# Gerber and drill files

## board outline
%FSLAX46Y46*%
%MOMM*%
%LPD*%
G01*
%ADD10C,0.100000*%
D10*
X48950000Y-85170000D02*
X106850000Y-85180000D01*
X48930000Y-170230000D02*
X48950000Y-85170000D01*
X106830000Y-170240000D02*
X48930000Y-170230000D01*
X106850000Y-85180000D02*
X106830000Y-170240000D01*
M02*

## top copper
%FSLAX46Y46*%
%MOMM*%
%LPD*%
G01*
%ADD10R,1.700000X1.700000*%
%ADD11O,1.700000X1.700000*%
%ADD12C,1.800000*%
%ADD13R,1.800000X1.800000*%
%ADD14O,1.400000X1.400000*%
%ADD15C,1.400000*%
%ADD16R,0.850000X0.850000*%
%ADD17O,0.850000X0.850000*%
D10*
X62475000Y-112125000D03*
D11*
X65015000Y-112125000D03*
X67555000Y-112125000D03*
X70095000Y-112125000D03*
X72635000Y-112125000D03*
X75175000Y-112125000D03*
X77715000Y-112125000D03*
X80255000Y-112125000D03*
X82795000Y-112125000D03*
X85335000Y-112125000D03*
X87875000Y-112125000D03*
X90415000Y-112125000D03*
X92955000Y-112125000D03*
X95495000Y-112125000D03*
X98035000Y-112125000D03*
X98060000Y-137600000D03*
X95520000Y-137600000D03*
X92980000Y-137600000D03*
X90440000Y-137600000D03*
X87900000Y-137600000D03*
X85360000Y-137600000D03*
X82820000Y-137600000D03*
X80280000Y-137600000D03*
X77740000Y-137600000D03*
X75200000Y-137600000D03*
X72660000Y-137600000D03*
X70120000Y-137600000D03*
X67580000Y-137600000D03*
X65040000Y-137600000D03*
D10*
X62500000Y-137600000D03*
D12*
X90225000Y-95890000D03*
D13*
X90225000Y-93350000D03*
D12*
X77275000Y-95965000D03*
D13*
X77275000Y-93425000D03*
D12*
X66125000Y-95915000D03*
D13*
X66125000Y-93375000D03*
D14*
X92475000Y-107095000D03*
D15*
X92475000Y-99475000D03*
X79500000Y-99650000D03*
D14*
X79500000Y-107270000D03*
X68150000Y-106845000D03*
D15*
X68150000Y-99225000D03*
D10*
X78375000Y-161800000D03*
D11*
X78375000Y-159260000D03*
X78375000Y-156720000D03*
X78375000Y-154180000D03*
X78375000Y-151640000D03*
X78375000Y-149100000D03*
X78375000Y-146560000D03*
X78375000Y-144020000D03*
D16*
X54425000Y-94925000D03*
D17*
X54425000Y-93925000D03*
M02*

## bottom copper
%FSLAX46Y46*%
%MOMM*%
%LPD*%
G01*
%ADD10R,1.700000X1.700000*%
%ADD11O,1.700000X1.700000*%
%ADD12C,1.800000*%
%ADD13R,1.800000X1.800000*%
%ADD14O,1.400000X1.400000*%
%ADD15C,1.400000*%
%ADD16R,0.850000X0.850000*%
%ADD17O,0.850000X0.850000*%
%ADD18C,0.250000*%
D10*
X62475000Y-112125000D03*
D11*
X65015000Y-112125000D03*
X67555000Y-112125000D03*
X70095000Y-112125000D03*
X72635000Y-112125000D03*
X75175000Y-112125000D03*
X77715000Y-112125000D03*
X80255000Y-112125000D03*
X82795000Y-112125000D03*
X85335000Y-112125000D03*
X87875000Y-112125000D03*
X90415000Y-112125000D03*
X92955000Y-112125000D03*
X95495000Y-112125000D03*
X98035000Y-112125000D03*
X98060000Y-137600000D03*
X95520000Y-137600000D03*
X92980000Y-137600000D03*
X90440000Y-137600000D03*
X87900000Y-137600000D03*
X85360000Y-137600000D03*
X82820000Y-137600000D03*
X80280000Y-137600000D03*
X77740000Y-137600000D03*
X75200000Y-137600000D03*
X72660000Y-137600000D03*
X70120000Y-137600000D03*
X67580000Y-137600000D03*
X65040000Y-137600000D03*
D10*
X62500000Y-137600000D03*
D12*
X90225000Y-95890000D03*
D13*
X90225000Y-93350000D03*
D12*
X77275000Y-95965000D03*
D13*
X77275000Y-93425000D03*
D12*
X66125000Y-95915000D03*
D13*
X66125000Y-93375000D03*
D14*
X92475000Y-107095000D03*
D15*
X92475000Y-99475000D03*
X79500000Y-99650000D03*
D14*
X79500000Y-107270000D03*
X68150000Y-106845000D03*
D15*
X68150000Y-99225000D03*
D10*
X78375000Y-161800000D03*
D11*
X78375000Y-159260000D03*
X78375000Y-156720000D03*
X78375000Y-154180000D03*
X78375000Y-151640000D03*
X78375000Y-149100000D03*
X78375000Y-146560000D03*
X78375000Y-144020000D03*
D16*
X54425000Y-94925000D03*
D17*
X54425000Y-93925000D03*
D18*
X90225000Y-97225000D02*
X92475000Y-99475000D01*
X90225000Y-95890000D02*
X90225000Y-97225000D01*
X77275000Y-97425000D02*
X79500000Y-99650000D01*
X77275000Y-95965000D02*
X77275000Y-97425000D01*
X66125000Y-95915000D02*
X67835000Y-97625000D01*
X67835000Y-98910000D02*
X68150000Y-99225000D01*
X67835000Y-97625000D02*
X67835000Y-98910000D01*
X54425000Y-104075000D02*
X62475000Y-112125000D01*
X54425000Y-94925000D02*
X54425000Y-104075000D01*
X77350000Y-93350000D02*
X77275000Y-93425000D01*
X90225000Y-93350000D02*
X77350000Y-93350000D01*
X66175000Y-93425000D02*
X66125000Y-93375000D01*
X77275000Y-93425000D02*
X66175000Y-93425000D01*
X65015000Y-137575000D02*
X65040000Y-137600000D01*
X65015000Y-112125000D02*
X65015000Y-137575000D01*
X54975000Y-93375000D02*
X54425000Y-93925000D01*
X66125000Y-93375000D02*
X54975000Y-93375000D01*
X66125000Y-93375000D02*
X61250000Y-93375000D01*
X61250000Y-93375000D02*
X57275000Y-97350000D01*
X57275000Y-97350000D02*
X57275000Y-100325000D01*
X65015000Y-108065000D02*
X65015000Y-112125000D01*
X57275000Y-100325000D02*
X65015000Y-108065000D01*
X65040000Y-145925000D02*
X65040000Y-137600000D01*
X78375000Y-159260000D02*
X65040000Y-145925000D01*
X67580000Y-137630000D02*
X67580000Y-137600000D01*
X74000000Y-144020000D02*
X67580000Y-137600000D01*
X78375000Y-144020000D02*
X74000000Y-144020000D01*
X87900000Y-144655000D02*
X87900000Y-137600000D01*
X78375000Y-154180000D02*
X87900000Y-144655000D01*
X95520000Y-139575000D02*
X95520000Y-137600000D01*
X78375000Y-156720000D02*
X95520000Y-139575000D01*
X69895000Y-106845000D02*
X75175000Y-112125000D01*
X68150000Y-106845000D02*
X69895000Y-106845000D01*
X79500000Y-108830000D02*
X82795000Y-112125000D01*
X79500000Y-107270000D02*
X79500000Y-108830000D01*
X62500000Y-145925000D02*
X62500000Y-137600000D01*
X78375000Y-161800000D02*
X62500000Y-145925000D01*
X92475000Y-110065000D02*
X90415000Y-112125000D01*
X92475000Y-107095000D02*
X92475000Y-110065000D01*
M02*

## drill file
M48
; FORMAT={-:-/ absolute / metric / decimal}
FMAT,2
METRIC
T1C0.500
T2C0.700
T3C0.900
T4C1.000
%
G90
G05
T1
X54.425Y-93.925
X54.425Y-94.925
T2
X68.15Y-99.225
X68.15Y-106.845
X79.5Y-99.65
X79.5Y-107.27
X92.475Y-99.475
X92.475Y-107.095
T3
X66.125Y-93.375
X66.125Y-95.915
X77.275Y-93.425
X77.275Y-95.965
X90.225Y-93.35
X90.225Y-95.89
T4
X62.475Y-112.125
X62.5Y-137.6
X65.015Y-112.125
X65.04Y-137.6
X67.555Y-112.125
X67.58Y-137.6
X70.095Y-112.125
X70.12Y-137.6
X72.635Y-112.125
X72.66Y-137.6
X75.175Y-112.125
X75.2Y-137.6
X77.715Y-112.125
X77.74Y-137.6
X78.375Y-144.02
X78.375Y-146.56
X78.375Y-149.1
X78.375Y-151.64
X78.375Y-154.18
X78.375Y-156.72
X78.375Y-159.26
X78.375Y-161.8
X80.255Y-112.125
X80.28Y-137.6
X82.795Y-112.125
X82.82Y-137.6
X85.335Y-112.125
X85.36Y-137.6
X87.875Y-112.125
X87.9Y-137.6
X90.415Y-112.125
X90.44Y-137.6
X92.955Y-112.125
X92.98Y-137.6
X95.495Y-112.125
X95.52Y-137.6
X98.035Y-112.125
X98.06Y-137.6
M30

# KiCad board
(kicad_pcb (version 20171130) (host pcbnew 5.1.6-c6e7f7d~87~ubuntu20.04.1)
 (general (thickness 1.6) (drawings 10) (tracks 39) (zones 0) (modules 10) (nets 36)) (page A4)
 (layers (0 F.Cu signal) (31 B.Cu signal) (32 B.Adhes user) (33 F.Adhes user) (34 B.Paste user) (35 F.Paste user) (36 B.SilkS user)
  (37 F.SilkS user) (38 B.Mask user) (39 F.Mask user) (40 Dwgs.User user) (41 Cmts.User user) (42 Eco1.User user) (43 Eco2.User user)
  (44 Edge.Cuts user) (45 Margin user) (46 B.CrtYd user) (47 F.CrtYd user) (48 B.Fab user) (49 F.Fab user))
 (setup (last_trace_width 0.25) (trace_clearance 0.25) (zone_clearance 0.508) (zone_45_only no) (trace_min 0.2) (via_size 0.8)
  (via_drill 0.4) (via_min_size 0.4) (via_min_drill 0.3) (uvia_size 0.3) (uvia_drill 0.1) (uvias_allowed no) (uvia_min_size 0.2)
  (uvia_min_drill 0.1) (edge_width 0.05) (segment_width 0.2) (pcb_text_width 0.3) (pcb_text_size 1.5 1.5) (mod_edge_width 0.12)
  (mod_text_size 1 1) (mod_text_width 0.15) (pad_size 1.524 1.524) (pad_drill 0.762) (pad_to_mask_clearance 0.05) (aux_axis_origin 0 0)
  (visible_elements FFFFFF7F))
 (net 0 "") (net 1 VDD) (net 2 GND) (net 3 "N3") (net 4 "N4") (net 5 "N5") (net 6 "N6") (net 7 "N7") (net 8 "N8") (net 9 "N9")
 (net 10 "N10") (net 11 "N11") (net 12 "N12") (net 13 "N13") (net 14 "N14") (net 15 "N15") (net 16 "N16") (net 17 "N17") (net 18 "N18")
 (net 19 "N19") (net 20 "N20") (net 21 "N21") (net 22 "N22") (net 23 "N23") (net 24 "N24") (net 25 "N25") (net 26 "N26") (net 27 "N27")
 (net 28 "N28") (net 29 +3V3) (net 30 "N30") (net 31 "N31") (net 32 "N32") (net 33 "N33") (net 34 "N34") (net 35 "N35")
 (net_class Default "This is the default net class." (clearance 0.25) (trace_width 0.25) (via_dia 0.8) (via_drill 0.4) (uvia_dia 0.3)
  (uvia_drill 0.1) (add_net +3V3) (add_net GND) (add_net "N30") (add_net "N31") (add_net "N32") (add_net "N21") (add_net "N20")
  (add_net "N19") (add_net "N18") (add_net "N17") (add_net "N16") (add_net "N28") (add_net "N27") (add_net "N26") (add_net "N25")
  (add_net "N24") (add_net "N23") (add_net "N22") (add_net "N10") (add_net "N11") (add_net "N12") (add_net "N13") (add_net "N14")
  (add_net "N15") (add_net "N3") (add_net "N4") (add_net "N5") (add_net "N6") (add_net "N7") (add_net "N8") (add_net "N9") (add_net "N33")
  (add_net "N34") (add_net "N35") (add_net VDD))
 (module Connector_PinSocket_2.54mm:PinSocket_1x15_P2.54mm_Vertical (layer F.Cu) (at 62.475 112.125 90)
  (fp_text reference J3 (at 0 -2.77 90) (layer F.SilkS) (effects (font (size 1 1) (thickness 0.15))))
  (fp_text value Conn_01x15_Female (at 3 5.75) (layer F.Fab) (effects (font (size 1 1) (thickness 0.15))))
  (pad 1 thru_hole rect (at 0 0 90) (size 1.7 1.7) (drill 1) (layers *.Cu *.Mask) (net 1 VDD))
  (pad 2 thru_hole oval (at 0 2.54 90) (size 1.7 1.7) (drill 1) (layers *.Cu *.Mask) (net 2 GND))
  (pad 3 thru_hole oval (at 0 5.08 90) (size 1.7 1.7) (drill 1) (layers *.Cu *.Mask) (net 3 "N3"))
  (pad 4 thru_hole oval (at 0 7.62 90) (size 1.7 1.7) (drill 1) (layers *.Cu *.Mask) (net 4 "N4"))
  (pad 5 thru_hole oval (at 0 10.16 90) (size 1.7 1.7) (drill 1) (layers *.Cu *.Mask) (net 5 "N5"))
  (pad 6 thru_hole oval (at 0 12.7 90) (size 1.7 1.7) (drill 1) (layers *.Cu *.Mask) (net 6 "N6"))
  (pad 7 thru_hole oval (at 0 15.24 90) (size 1.7 1.7) (drill 1) (layers *.Cu *.Mask) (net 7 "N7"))
  (pad 8 thru_hole oval (at 0 17.78 90) (size 1.7 1.7) (drill 1) (layers *.Cu *.Mask) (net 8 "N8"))
  (pad 9 thru_hole oval (at 0 20.32 90) (size 1.7 1.7) (drill 1) (layers *.Cu *.Mask) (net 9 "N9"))
  (pad 10 thru_hole oval (at 0 22.86 90) (size 1.7 1.7) (drill 1) (layers *.Cu *.Mask) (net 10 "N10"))
  (pad 11 thru_hole oval (at 0 25.4 90) (size 1.7 1.7) (drill 1) (layers *.Cu *.Mask) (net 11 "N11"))
  (pad 12 thru_hole oval (at 0 27.94 90) (size 1.7 1.7) (drill 1) (layers *.Cu *.Mask) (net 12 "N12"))
  (pad 13 thru_hole oval (at 0 30.48 90) (size 1.7 1.7) (drill 1) (layers *.Cu *.Mask) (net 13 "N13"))
  (pad 14 thru_hole oval (at 0 33.02 90) (size 1.7 1.7) (drill 1) (layers *.Cu *.Mask) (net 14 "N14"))
  (pad 15 thru_hole oval (at 0 35.56 90) (size 1.7 1.7) (drill 1) (layers *.Cu *.Mask) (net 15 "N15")))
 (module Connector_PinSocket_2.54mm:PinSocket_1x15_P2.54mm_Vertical (layer F.Cu) (at 62.5 137.6 90)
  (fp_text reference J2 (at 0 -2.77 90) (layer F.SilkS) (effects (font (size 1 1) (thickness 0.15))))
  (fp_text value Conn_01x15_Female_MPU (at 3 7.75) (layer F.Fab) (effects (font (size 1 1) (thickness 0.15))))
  (pad 15 thru_hole oval (at 0 35.56 90) (size 1.7 1.7) (drill 1) (layers *.Cu *.Mask) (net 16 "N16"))
  (pad 14 thru_hole oval (at 0 33.02 90) (size 1.7 1.7) (drill 1) (layers *.Cu *.Mask) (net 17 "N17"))
  (pad 13 thru_hole oval (at 0 30.48 90) (size 1.7 1.7) (drill 1) (layers *.Cu *.Mask) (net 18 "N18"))
  (pad 12 thru_hole oval (at 0 27.94 90) (size 1.7 1.7) (drill 1) (layers *.Cu *.Mask) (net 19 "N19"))
  (pad 11 thru_hole oval (at 0 25.4 90) (size 1.7 1.7) (drill 1) (layers *.Cu *.Mask) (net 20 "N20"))
  (pad 10 thru_hole oval (at 0 22.86 90) (size 1.7 1.7) (drill 1) (layers *.Cu *.Mask) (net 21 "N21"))
  (pad 9 thru_hole oval (at 0 20.32 90) (size 1.7 1.7) (drill 1) (layers *.Cu *.Mask) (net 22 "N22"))
  (pad 8 thru_hole oval (at 0 17.78 90) (size 1.7 1.7) (drill 1) (layers *.Cu *.Mask) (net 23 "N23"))
  (pad 7 thru_hole oval (at 0 15.24 90) (size 1.7 1.7) (drill 1) (layers *.Cu *.Mask) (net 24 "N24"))
  (pad 6 thru_hole oval (at 0 12.7 90) (size 1.7 1.7) (drill 1) (layers *.Cu *.Mask) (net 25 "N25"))
  (pad 5 thru_hole oval (at 0 10.16 90) (size 1.7 1.7) (drill 1) (layers *.Cu *.Mask) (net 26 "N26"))
  (pad 4 thru_hole oval (at 0 7.62 90) (size 1.7 1.7) (drill 1) (layers *.Cu *.Mask) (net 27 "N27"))
  (pad 3 thru_hole oval (at 0 5.08 90) (size 1.7 1.7) (drill 1) (layers *.Cu *.Mask) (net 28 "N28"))
  (pad 2 thru_hole oval (at 0 2.54 90) (size 1.7 1.7) (drill 1) (layers *.Cu *.Mask) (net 2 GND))
  (pad 1 thru_hole rect (at 0 0 90) (size 1.7 1.7) (drill 1) (layers *.Cu *.Mask) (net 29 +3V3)))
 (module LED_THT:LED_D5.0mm (layer F.Cu) (at 90.225 93.35 270)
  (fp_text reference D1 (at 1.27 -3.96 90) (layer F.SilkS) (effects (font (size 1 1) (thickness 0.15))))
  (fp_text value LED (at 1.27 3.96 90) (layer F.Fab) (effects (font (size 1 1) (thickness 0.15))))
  (pad 2 thru_hole circle (at 2.54 0 270) (size 1.8 1.8) (drill 0.9) (layers *.Cu *.Mask) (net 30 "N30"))
  (pad 1 thru_hole rect (at 0 0 270) (size 1.8 1.8) (drill 0.9) (layers *.Cu *.Mask) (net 2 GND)))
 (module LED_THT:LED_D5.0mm (layer F.Cu) (at 77.275 93.425 270)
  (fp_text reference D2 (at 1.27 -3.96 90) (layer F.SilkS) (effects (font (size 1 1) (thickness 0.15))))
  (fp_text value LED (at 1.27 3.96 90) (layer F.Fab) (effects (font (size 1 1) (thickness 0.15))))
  (pad 2 thru_hole circle (at 2.54 0 270) (size 1.8 1.8) (drill 0.9) (layers *.Cu *.Mask) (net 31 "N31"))
  (pad 1 thru_hole rect (at 0 0 270) (size 1.8 1.8) (drill 0.9) (layers *.Cu *.Mask) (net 2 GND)))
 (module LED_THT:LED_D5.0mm (layer F.Cu) (at 66.125 93.375 270)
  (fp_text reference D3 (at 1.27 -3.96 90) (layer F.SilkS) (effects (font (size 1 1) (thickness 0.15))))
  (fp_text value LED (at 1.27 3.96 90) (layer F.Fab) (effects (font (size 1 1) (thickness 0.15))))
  (pad 2 thru_hole circle (at 2.54 0 270) (size 1.8 1.8) (drill 0.9) (layers *.Cu *.Mask) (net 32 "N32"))
  (pad 1 thru_hole rect (at 0 0 270) (size 1.8 1.8) (drill 0.9) (layers *.Cu *.Mask) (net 2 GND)))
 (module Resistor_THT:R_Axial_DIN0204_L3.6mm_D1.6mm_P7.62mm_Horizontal (layer F.Cu) (at 92.475 99.475 270)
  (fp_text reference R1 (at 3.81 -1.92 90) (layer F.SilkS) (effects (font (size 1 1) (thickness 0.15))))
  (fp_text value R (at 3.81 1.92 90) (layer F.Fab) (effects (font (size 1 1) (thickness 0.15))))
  (pad 2 thru_hole oval (at 7.62 0 270) (size 1.4 1.4) (drill 0.7) (layers *.Cu *.Mask) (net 12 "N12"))
  (pad 1 thru_hole circle (at 0 0 270) (size 1.4 1.4) (drill 0.7) (layers *.Cu *.Mask) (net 30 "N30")))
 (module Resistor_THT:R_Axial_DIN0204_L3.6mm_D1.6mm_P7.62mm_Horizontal (layer F.Cu) (at 79.5 99.65 270)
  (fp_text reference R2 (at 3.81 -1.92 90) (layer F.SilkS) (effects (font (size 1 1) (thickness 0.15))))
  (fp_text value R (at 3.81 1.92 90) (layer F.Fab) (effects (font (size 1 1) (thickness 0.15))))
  (pad 1 thru_hole circle (at 0 0 270) (size 1.4 1.4) (drill 0.7) (layers *.Cu *.Mask) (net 31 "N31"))
  (pad 2 thru_hole oval (at 7.62 0 270) (size 1.4 1.4) (drill 0.7) (layers *.Cu *.Mask) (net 9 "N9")))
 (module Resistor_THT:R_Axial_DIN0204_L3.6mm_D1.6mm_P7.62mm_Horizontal (layer F.Cu) (at 68.15 99.225 270)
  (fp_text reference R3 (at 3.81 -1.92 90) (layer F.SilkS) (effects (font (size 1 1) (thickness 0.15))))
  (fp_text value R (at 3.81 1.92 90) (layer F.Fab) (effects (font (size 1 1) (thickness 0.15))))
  (pad 2 thru_hole oval (at 7.62 0 270) (size 1.4 1.4) (drill 0.7) (layers *.Cu *.Mask) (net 6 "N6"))
  (pad 1 thru_hole circle (at 0 0 270) (size 1.4 1.4) (drill 0.7) (layers *.Cu *.Mask) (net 32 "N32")))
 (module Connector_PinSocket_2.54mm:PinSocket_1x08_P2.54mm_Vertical (layer F.Cu) (at 78.375 161.8 180)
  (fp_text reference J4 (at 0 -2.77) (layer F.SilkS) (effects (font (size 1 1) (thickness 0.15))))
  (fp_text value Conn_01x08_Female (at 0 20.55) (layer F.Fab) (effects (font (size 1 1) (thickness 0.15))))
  (pad 1 thru_hole rect (at 0 0 180) (size 1.7 1.7) (drill 1) (layers *.Cu *.Mask) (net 29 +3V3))
  (pad 2 thru_hole oval (at 0 2.54 180) (size 1.7 1.7) (drill 1) (layers *.Cu *.Mask) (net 2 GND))
  (pad 3 thru_hole oval (at 0 5.08 180) (size 1.7 1.7) (drill 1) (layers *.Cu *.Mask) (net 17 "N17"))
  (pad 4 thru_hole oval (at 0 7.62 180) (size 1.7 1.7) (drill 1) (layers *.Cu *.Mask) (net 20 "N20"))
  (pad 5 thru_hole oval (at 0 10.16 180) (size 1.7 1.7) (drill 1) (layers *.Cu *.Mask) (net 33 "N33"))
  (pad 6 thru_hole oval (at 0 12.7 180) (size 1.7 1.7) (drill 1) (layers *.Cu *.Mask) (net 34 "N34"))
  (pad 7 thru_hole oval (at 0 15.24 180) (size 1.7 1.7) (drill 1) (layers *.Cu *.Mask) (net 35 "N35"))
  (pad 8 thru_hole oval (at 0 17.78 180) (size 1.7 1.7) (drill 1) (layers *.Cu *.Mask) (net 28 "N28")))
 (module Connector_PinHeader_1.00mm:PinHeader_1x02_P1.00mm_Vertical (layer F.Cu) (at 54.425 94.925 180)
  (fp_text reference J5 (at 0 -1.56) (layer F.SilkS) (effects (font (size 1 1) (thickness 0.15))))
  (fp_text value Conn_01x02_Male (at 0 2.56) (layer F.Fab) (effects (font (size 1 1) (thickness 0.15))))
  (pad 1 thru_hole rect (at 0 0 180) (size 0.85 0.85) (drill 0.5) (layers *.Cu *.Mask) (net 1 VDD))
  (pad 2 thru_hole oval (at 0 1 180) (size 0.85 0.85) (drill 0.5) (layers *.Cu *.Mask) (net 2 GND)))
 (gr_line (start 48.95 85.17) (end 106.85 85.18) (layer Edge.Cuts) (width 0.1))
 (gr_line (start 48.93 170.23) (end 48.95 85.17) (layer Edge.Cuts) (width 0.1))
 (gr_line (start 106.83 170.24) (end 48.93 170.23) (layer Edge.Cuts) (width 0.1))
 (gr_line (start 106.85 85.18) (end 106.83 170.24) (layer Edge.Cuts) (width 0.1))
 (segment (start 90.225 97.225) (end 92.475 99.475) (width 0.25) (layer B.Cu) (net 30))
 (segment (start 90.225 95.89) (end 90.225 97.225) (width 0.25) (layer B.Cu) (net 30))
 (segment (start 77.275 97.425) (end 79.5 99.65) (width 0.25) (layer B.Cu) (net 31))
 (segment (start 77.275 95.965) (end 77.275 97.425) (width 0.25) (layer B.Cu) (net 31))
 (segment (start 66.125 95.915) (end 67.835 97.625) (width 0.25) (layer B.Cu) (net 32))
 (segment (start 67.835 98.91) (end 68.15 99.225) (width 0.25) (layer B.Cu) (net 32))
 (segment (start 67.835 97.625) (end 67.835 98.91) (width 0.25) (layer B.Cu) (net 32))
 (segment (start 54.425 104.075) (end 62.475 112.125) (width 0.25) (layer B.Cu) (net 1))
 (segment (start 54.425 94.925) (end 54.425 104.075) (width 0.25) (layer B.Cu) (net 1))
 (segment (start 77.35 93.35) (end 77.275 93.425) (width 0.25) (layer B.Cu) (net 2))
 (segment (start 90.225 93.35) (end 77.35 93.35) (width 0.25) (layer B.Cu) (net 2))
 (segment (start 66.175 93.425) (end 66.125 93.375) (width 0.25) (layer B.Cu) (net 2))
 (segment (start 77.275 93.425) (end 66.175 93.425) (width 0.25) (layer B.Cu) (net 2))
 (segment (start 65.015 137.575) (end 65.04 137.6) (width 0.25) (layer B.Cu) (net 2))
 (segment (start 65.015 112.125) (end 65.015 137.575) (width 0.25) (layer B.Cu) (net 2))
 (segment (start 54.975 93.375) (end 54.425 93.925) (width 0.25) (layer B.Cu) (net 2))
 (segment (start 66.125 93.375) (end 54.975 93.375) (width 0.25) (layer B.Cu) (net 2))
 (segment (start 66.125 93.375) (end 61.25 93.375) (width 0.25) (layer B.Cu) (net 2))
 (segment (start 61.25 93.375) (end 57.275 97.35) (width 0.25) (layer B.Cu) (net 2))
 (segment (start 57.275 97.35) (end 57.275 100.325) (width 0.25) (layer B.Cu) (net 2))
 (segment (start 65.015 108.065) (end 65.015 112.125) (width 0.25) (layer B.Cu) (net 2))
 (segment (start 57.275 100.325) (end 65.015 108.065) (width 0.25) (layer B.Cu) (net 2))
 (segment (start 65.04 145.925) (end 65.04 137.6) (width 0.25) (layer B.Cu) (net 2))
 (segment (start 78.375 159.26) (end 65.04 145.925) (width 0.25) (layer B.Cu) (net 2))
 (segment (start 67.58 137.63) (end 67.58 137.6) (width 0.25) (layer B.Cu) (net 28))
 (segment (start 74 144.02) (end 67.58 137.6) (width 0.25) (layer B.Cu) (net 28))
 (segment (start 78.375 144.02) (end 74 144.02) (width 0.25) (layer B.Cu) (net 28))
 (segment (start 87.9 144.655) (end 87.9 137.6) (width 0.25) (layer B.Cu) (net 20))
 (segment (start 78.375 154.18) (end 87.9 144.655) (width 0.25) (layer B.Cu) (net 20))
 (segment (start 95.52 139.575) (end 95.52 137.6) (width 0.25) (layer B.Cu) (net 17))
 (segment (start 78.375 156.72) (end 95.52 139.575) (width 0.25) (layer B.Cu) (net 17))
 (segment (start 69.895 106.845) (end 75.175 112.125) (width 0.25) (layer B.Cu) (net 6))
 (segment (start 68.15 106.845) (end 69.895 106.845) (width 0.25) (layer B.Cu) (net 6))
 (segment (start 79.5 108.83) (end 82.795 112.125) (width 0.25) (layer B.Cu) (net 9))
 (segment (start 79.5 107.27) (end 79.5 108.83) (width 0.25) (layer B.Cu) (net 9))
 (segment (start 62.5 145.925) (end 62.5 137.6) (width 0.25) (layer B.Cu) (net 29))
 (segment (start 78.375 161.8) (end 62.5 145.925) (width 0.25) (layer B.Cu) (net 29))
 (segment (start 92.475 110.065) (end 90.415 112.125) (width 0.25) (layer B.Cu) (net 12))
 (segment (start 92.475 107.095) (end 92.475 110.065) (width 0.25) (layer B.Cu) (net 12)))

